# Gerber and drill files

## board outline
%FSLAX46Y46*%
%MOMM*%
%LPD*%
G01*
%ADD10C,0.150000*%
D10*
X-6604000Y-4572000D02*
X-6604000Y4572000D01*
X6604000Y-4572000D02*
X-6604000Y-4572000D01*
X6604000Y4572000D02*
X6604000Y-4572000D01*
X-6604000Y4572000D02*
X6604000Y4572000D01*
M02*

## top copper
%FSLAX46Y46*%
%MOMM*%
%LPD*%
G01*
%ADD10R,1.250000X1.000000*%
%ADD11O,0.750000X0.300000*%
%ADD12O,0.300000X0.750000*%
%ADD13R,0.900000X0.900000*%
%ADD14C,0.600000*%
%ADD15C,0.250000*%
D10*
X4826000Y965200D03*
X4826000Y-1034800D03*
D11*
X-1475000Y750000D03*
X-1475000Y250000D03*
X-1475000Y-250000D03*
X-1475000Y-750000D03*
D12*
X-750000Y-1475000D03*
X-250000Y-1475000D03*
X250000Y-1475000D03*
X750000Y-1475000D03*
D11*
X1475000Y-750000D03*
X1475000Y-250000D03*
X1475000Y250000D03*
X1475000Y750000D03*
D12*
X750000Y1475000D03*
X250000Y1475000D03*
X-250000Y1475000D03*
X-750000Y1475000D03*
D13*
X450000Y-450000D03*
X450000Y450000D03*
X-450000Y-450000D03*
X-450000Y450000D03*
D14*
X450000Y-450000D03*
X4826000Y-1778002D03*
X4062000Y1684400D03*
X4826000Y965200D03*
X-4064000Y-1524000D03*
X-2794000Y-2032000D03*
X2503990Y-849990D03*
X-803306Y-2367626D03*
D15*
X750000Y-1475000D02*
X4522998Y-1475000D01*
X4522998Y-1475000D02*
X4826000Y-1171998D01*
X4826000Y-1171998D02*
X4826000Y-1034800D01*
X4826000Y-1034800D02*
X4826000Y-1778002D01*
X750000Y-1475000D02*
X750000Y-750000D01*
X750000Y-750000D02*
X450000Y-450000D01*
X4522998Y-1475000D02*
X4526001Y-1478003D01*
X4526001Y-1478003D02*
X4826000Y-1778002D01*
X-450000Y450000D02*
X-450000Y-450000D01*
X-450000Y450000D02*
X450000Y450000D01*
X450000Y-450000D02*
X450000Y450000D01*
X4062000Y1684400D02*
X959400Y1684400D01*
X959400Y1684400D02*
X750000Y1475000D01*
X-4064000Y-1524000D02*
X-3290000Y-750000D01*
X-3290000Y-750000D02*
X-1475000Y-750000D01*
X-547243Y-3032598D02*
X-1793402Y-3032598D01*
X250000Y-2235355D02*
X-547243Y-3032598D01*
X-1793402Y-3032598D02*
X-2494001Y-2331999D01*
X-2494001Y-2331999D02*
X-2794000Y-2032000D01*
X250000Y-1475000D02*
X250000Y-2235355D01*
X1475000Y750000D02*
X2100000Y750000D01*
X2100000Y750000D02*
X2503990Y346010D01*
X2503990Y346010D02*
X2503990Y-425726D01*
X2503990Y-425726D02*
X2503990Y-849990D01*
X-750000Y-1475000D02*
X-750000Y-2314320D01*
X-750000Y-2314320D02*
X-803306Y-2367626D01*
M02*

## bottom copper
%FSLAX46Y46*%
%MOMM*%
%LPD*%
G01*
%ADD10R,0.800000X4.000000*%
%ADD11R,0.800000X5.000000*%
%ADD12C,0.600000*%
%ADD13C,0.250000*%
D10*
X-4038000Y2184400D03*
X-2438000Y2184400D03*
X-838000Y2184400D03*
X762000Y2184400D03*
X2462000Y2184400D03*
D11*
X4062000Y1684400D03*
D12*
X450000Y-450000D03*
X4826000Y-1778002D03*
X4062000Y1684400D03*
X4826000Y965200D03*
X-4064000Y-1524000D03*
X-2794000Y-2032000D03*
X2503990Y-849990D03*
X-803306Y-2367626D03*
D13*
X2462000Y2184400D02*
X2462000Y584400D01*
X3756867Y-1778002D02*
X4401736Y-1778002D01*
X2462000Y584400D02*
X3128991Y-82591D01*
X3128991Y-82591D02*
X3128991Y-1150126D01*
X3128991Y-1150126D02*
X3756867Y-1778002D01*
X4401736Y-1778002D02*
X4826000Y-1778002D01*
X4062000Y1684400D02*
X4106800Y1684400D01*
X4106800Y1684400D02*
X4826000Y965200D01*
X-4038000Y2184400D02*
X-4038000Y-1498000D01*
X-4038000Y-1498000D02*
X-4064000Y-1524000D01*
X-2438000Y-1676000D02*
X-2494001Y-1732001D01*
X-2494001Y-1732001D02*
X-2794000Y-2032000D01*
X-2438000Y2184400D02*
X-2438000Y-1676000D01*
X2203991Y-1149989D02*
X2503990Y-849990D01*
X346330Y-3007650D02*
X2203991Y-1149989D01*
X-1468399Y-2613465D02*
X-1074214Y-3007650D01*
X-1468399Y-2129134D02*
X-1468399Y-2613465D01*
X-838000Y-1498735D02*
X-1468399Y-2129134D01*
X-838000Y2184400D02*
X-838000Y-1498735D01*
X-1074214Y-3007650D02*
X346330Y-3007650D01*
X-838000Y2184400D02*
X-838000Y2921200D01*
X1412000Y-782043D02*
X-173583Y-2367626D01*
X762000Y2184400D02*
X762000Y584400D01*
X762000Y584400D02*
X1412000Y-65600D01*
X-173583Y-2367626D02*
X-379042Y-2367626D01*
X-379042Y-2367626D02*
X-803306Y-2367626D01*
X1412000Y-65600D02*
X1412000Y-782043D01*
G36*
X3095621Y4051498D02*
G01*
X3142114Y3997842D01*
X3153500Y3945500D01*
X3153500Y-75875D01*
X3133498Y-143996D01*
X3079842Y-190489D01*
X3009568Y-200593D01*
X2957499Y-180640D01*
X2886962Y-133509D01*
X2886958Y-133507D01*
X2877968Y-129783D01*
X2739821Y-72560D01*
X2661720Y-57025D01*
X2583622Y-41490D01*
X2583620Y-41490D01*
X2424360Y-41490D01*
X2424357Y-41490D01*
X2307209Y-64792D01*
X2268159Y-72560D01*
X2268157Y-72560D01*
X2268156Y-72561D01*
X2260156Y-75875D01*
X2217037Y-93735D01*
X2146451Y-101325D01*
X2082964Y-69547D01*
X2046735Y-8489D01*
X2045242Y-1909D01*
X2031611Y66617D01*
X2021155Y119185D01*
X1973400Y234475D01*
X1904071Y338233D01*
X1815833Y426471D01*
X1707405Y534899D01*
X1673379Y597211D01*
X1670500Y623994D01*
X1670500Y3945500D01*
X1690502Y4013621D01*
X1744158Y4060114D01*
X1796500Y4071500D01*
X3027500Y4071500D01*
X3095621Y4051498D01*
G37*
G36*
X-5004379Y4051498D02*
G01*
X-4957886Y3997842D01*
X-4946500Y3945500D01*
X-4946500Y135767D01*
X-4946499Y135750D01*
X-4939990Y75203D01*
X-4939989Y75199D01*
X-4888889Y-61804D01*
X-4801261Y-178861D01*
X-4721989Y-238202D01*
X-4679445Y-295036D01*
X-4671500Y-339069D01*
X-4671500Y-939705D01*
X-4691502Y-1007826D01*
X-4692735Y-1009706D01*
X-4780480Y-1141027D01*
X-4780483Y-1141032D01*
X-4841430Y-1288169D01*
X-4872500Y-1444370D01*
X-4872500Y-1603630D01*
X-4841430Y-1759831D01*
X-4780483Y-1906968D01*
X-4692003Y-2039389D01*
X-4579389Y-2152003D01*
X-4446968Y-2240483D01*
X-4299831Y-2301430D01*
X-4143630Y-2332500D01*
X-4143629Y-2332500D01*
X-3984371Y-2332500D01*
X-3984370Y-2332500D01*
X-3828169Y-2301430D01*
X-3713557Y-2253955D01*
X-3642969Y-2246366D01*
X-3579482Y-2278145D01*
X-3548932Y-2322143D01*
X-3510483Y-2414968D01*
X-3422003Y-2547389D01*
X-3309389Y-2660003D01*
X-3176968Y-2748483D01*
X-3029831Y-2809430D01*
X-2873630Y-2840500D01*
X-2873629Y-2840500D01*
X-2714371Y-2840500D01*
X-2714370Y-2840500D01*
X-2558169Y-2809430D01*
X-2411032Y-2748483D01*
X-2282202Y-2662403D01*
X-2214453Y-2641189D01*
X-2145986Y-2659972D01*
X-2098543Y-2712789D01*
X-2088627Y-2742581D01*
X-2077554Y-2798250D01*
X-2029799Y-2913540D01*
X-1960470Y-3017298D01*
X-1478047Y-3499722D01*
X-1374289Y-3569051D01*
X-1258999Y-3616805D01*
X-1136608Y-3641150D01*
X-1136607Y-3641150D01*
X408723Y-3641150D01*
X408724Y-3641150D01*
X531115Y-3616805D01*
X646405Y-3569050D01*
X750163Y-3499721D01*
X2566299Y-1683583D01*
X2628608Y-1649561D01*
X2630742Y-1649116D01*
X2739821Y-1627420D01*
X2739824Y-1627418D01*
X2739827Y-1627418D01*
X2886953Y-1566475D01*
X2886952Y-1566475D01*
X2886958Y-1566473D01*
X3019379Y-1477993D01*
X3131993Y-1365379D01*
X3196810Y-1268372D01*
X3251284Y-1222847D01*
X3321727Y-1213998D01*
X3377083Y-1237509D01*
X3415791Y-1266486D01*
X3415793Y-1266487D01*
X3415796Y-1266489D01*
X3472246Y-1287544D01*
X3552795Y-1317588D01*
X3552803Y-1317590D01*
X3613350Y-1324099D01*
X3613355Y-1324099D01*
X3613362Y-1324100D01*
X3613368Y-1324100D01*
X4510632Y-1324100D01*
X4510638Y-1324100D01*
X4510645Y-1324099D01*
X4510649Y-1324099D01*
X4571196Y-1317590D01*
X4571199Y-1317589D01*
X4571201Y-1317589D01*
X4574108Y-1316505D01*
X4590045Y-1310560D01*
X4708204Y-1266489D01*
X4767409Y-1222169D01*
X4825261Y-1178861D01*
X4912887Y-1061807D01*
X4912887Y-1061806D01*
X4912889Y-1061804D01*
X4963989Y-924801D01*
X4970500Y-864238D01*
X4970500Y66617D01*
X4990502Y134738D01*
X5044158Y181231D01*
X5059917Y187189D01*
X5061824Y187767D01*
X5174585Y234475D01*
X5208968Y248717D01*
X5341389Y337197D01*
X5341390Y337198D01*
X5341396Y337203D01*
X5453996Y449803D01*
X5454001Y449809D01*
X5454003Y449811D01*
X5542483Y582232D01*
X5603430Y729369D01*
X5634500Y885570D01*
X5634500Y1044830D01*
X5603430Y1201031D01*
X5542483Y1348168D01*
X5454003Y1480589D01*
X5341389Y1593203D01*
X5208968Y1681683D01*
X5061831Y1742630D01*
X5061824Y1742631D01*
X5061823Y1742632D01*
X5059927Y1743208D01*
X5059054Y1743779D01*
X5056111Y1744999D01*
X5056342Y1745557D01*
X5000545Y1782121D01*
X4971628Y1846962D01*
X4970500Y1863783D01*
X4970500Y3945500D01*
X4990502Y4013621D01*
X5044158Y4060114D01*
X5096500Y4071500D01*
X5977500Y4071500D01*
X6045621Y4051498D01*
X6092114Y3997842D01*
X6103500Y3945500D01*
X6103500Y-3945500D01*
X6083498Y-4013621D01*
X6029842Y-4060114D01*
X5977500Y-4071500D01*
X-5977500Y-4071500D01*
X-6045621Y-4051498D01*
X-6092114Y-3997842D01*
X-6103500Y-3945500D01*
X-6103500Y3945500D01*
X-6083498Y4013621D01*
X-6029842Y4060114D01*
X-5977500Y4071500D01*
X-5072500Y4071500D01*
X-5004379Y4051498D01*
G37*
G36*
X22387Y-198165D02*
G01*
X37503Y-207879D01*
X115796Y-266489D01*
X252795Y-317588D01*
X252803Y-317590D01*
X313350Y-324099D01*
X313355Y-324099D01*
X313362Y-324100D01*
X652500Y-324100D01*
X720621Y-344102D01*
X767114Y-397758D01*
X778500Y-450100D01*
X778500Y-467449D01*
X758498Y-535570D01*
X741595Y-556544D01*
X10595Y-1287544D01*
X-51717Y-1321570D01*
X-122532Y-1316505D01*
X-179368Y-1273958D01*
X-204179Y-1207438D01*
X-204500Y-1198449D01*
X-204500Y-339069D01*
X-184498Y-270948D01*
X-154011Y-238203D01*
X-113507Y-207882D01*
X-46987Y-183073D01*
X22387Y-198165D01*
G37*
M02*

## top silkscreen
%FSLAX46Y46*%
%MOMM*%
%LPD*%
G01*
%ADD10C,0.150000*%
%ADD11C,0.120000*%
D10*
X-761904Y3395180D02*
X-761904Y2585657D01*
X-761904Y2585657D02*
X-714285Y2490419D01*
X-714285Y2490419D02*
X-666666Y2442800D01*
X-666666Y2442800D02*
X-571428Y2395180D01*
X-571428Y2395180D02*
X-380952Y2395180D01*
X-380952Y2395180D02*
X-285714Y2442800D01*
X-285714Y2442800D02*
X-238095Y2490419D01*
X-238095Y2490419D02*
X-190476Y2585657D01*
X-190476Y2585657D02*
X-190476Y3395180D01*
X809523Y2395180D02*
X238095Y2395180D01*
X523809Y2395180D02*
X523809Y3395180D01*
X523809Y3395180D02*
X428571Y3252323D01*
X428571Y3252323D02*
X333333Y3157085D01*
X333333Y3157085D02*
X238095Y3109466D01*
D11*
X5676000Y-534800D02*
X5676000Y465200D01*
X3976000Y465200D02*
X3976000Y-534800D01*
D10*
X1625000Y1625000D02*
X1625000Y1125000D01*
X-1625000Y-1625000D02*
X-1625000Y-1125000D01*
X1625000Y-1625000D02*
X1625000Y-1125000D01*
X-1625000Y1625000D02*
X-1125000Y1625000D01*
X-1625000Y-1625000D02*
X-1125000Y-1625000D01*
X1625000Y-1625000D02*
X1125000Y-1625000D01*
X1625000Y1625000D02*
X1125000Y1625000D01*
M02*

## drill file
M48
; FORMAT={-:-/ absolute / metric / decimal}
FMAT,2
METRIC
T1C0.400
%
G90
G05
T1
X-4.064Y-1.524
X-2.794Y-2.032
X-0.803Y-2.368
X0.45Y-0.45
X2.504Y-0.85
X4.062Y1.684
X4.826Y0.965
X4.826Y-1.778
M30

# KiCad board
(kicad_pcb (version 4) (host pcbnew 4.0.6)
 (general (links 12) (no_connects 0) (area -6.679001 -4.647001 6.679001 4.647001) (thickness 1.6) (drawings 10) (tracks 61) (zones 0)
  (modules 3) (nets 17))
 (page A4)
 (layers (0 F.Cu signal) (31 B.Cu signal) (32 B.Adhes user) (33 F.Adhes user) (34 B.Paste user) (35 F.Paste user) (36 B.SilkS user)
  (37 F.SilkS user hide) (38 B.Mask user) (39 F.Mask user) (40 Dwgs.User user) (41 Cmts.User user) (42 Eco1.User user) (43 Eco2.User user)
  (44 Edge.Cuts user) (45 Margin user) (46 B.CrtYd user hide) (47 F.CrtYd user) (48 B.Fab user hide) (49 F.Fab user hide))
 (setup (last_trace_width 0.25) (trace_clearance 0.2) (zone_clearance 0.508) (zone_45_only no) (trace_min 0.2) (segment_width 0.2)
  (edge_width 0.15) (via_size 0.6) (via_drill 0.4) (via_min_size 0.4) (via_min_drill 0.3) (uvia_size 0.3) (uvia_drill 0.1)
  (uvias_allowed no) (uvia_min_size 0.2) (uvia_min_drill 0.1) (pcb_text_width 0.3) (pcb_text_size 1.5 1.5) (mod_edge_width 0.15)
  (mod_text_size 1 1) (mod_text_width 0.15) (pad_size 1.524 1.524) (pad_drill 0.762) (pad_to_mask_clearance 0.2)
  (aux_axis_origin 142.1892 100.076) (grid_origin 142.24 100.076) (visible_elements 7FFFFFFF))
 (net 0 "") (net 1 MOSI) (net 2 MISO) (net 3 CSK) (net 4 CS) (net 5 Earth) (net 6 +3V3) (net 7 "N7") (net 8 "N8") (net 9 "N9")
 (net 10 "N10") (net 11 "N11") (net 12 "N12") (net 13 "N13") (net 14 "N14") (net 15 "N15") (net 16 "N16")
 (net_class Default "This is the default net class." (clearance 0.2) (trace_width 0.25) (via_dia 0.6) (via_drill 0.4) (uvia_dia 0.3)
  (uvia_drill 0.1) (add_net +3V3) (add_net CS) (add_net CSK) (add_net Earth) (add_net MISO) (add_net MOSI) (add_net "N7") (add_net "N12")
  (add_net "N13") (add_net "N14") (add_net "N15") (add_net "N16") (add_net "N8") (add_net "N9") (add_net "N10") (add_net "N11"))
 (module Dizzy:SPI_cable (layer B.Cu) (at -4.438 -0.1844)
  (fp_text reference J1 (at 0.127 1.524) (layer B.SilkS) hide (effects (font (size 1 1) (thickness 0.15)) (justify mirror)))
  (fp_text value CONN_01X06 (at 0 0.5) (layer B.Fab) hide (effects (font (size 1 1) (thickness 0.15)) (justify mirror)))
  (pad 1 smd rect (at 0.4 -2) (size 0.8 4) (layers B.Cu B.Paste B.Mask) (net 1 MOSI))
  (pad 2 smd rect (at 2 -2) (size 0.8 4) (layers B.Cu B.Paste B.Mask) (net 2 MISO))
  (pad 3 smd rect (at 3.6 -2) (size 0.8 4) (layers B.Cu B.Paste B.Mask) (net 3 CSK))
  (pad 4 smd rect (at 5.2 -2) (size 0.8 4) (layers B.Cu B.Paste B.Mask) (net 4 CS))
  (pad 5 smd rect (at 6.9 -2) (size 0.8 4) (layers B.Cu B.Paste B.Mask) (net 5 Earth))
  (pad 6 smd rect (at 8.5 -1.5) (size 0.8 5) (layers B.Cu B.Paste B.Mask) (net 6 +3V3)))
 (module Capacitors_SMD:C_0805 (layer F.Cu) (at 4.826 0.0348 270)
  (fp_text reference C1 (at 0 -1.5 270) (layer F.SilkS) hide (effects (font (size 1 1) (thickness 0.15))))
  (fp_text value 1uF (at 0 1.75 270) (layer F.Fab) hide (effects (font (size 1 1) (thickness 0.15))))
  (fp_line (start 0.5 -0.85) (end -0.5 -0.85) (layer F.SilkS) (width 0.12))
  (fp_line (start -0.5 0.85) (end 0.5 0.85) (layer F.SilkS) (width 0.12))
  (pad 1 smd rect (at -1 0 270) (size 1 1.25) (layers F.Cu F.Paste F.Mask) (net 6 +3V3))
  (pad 2 smd rect (at 1 0 270) (size 1 1.25) (layers F.Cu F.Paste F.Mask) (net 5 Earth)))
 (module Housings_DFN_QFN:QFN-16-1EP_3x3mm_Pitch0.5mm (layer F.Cu) (at 0 0)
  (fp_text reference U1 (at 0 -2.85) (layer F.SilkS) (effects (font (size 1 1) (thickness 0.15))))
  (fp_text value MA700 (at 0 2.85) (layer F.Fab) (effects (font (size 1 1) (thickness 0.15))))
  (fp_line (start 1.625 -1.625) (end 1.625 -1.125) (layer F.SilkS) (width 0.15))
  (fp_line (start -1.625 1.625) (end -1.625 1.125) (layer F.SilkS) (width 0.15))
  (fp_line (start 1.625 1.625) (end 1.625 1.125) (layer F.SilkS) (width 0.15))
  (fp_line (start -1.625 -1.625) (end -1.125 -1.625) (layer F.SilkS) (width 0.15))
  (fp_line (start -1.625 1.625) (end -1.125 1.625) (layer F.SilkS) (width 0.15))
  (fp_line (start 1.625 1.625) (end 1.125 1.625) (layer F.SilkS) (width 0.15))
  (fp_line (start 1.625 -1.625) (end 1.125 -1.625) (layer F.SilkS) (width 0.15))
  (pad 1 smd oval (at -1.475 -0.75) (size 0.75 0.3) (layers F.Cu F.Paste F.Mask) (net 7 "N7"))
  (pad 2 smd oval (at -1.475 -0.25) (size 0.75 0.3) (layers F.Cu F.Paste F.Mask) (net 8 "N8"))
  (pad 3 smd oval (at -1.475 0.25) (size 0.75 0.3) (layers F.Cu F.Paste F.Mask) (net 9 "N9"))
  (pad 4 smd oval (at -1.475 0.75) (size 0.75 0.3) (layers F.Cu F.Paste F.Mask) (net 1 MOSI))
  (pad 5 smd oval (at -0.75 1.475 90) (size 0.75 0.3) (layers F.Cu F.Paste F.Mask) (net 4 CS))
  (pad 6 smd oval (at -0.25 1.475 90) (size 0.75 0.3) (layers F.Cu F.Paste F.Mask) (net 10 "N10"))
  (pad 7 smd oval (at 0.25 1.475 90) (size 0.75 0.3) (layers F.Cu F.Paste F.Mask) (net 2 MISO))
  (pad 8 smd oval (at 0.75 1.475 90) (size 0.75 0.3) (layers F.Cu F.Paste F.Mask) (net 5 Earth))
  (pad 9 smd oval (at 1.475 0.75) (size 0.75 0.3) (layers F.Cu F.Paste F.Mask) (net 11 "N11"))
  (pad 10 smd oval (at 1.475 0.25) (size 0.75 0.3) (layers F.Cu F.Paste F.Mask) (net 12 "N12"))
  (pad 11 smd oval (at 1.475 -0.25) (size 0.75 0.3) (layers F.Cu F.Paste F.Mask) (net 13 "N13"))
  (pad 12 smd oval (at 1.475 -0.75) (size 0.75 0.3) (layers F.Cu F.Paste F.Mask) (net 3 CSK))
  (pad 13 smd oval (at 0.75 -1.475 90) (size 0.75 0.3) (layers F.Cu F.Paste F.Mask) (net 6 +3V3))
  (pad 14 smd oval (at 0.25 -1.475 90) (size 0.75 0.3) (layers F.Cu F.Paste F.Mask) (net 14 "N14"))
  (pad 15 smd oval (at -0.25 -1.475 90) (size 0.75 0.3) (layers F.Cu F.Paste F.Mask) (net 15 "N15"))
  (pad 16 smd oval (at -0.75 -1.475 90) (size 0.75 0.3) (layers F.Cu F.Paste F.Mask) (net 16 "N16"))
  (pad 17 smd rect (at 0.45 0.45) (size 0.9 0.9) (layers F.Cu F.Paste F.Mask) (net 5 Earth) (solder_paste_margin_ratio -0.2))
  (pad 17 smd rect (at 0.45 -0.45) (size 0.9 0.9) (layers F.Cu F.Paste F.Mask) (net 5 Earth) (solder_paste_margin_ratio -0.2))
  (pad 17 smd rect (at -0.45 0.45) (size 0.9 0.9) (layers F.Cu F.Paste F.Mask) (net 5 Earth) (solder_paste_margin_ratio -0.2))
  (pad 17 smd rect (at -0.45 -0.45) (size 0.9 0.9) (layers F.Cu F.Paste F.Mask) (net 5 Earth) (solder_paste_margin_ratio -0.2)))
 (gr_line (start -6.604 4.572) (end -6.604 -4.572) (layer Edge.Cuts) (width 0.15))
 (gr_line (start 6.604 4.572) (end -6.604 4.572) (layer Edge.Cuts) (width 0.15))
 (gr_line (start 6.604 -4.572) (end 6.604 4.572) (layer Edge.Cuts) (width 0.15))
 (gr_line (start -6.604 -4.572) (end 6.604 -4.572) (layer Edge.Cuts) (width 0.15))
 (segment (start 0.75 1.475) (end 4.522998 1.475) (width 0.25) (layer F.Cu) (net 5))
 (segment (start 2.462 -2.1844) (end 2.462 -0.5844) (width 0.25) (layer B.Cu) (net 5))
 (segment (start 3.756867 1.778002) (end 4.401736 1.778002) (width 0.25) (layer B.Cu) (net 5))
 (segment (start 2.462 -0.5844) (end 3.128991 0.082591) (width 0.25) (layer B.Cu) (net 5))
 (segment (start 3.128991 0.082591) (end 3.128991 1.150126) (width 0.25) (layer B.Cu) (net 5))
 (segment (start 3.128991 1.150126) (end 3.756867 1.778002) (width 0.25) (layer B.Cu) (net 5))
 (segment (start 4.401736 1.778002) (end 4.826 1.778002) (width 0.25) (layer B.Cu) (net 5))
 (segment (start 4.522998 1.475) (end 4.826 1.171998) (width 0.25) (layer F.Cu) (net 5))
 (segment (start 4.826 1.171998) (end 4.826 1.0348) (width 0.25) (layer F.Cu) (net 5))
 (segment (start 4.826 1.0348) (end 4.826 1.778002) (width 0.25) (layer F.Cu) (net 5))
 (segment (start 0.75 1.475) (end 0.75 0.75) (width 0.25) (layer F.Cu) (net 5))
 (segment (start 0.75 0.75) (end 0.45 0.45) (width 0.25) (layer F.Cu) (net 5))
 (via (at 0.45 0.45) (size 0.6) (drill 0.4) (layers F.Cu B.Cu) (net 5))
 (segment (start 4.522998 1.475) (end 4.526001 1.478003) (width 0.25) (layer F.Cu) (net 5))
 (segment (start 4.526001 1.478003) (end 4.826 1.778002) (width 0.25) (layer F.Cu) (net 5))
 (via (at 4.826 1.778002) (size 0.6) (drill 0.4) (layers F.Cu B.Cu) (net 5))
 (segment (start -0.45 -0.45) (end -0.45 0.45) (width 0.25) (layer F.Cu) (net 5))
 (segment (start -0.45 -0.45) (end 0.45 -0.45) (width 0.25) (layer F.Cu) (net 5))
 (segment (start 0.45 0.45) (end 0.45 -0.45) (width 0.25) (layer F.Cu) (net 5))
 (segment (start 4.062 -1.6844) (end 0.9594 -1.6844) (width 0.25) (layer F.Cu) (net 6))
 (segment (start 0.9594 -1.6844) (end 0.75 -1.475) (width 0.25) (layer F.Cu) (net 6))
 (via (at 4.062 -1.6844) (size 0.6) (drill 0.4) (layers F.Cu B.Cu) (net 6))
 (segment (start 4.062 -1.6844) (end 4.1068 -1.6844) (width 0.25) (layer B.Cu) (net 6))
 (via (at 4.826 -0.9652) (size 0.6) (drill 0.4) (layers F.Cu B.Cu) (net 6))
 (segment (start 4.1068 -1.6844) (end 4.826 -0.9652) (width 0.25) (layer B.Cu) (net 6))
 (segment (start -4.064 1.524) (end -3.29 0.75) (width 0.25) (layer F.Cu) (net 1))
 (segment (start -3.29 0.75) (end -1.475 0.75) (width 0.25) (layer F.Cu) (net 1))
 (segment (start -4.038 -2.1844) (end -4.038 1.498) (width 0.25) (layer B.Cu) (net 1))
 (segment (start -4.038 1.498) (end -4.064 1.524) (width 0.25) (layer B.Cu) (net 1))
 (via (at -4.064 1.524) (size 0.6) (drill 0.4) (layers F.Cu B.Cu) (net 1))
 (segment (start -0.547243 3.032598) (end -1.793402 3.032598) (width 0.25) (layer F.Cu) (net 2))
 (segment (start 0.25 2.235355) (end -0.547243 3.032598) (width 0.25) (layer F.Cu) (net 2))
 (segment (start -1.793402 3.032598) (end -2.494001 2.331999) (width 0.25) (layer F.Cu) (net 2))
 (segment (start -2.494001 2.331999) (end -2.794 2.032) (width 0.25) (layer F.Cu) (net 2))
 (segment (start 0.25 1.475) (end 0.25 2.235355) (width 0.25) (layer F.Cu) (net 2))
 (segment (start -2.438 1.676) (end -2.494001 1.732001) (width 0.25) (layer B.Cu) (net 2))
 (segment (start -2.494001 1.732001) (end -2.794 2.032) (width 0.25) (layer B.Cu) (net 2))
 (segment (start -2.438 -2.1844) (end -2.438 1.676) (width 0.25) (layer B.Cu) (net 2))
 (via (at -2.794 2.032) (size 0.6) (drill 0.4) (layers F.Cu B.Cu) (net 2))
 (segment (start 1.475 -0.75) (end 2.1 -0.75) (width 0.25) (layer F.Cu) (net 3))
 (segment (start 2.203991 1.149989) (end 2.50399 0.84999) (width 0.25) (layer B.Cu) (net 3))
 (segment (start 0.34633 3.00765) (end 2.203991 1.149989) (width 0.25) (layer B.Cu) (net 3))
 (segment (start 2.1 -0.75) (end 2.50399 -0.34601) (width 0.25) (layer F.Cu) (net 3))
 (segment (start 2.50399 -0.34601) (end 2.50399 0.425726) (width 0.25) (layer F.Cu) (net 3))
 (segment (start -1.468399 2.613465) (end -1.074214 3.00765) (width 0.25) (layer B.Cu) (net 3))
 (segment (start -1.468399 2.129134) (end -1.468399 2.613465) (width 0.25) (layer B.Cu) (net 3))
 (segment (start -0.838 1.498735) (end -1.468399 2.129134) (width 0.25) (layer B.Cu) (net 3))
 (segment (start -0.838 -2.1844) (end -0.838 1.498735) (width 0.25) (layer B.Cu) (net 3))
 (segment (start -1.074214 3.00765) (end 0.34633 3.00765) (width 0.25) (layer B.Cu) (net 3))
 (segment (start 2.50399 0.425726) (end 2.50399 0.84999) (width 0.25) (layer F.Cu) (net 3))
 (via (at 2.50399 0.84999) (size 0.6) (drill 0.4) (layers F.Cu B.Cu) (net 3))
 (segment (start -0.838 -2.1844) (end -0.838 -2.9212) (width 0.25) (layer B.Cu) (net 3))
 (segment (start -0.75 1.475) (end -0.75 2.31432) (width 0.25) (layer F.Cu) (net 4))
 (segment (start -0.75 2.31432) (end -0.803306 2.367626) (width 0.25) (layer F.Cu) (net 4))
 (segment (start 1.412 0.782043) (end -0.173583 2.367626) (width 0.25) (layer B.Cu) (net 4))
 (via (at -0.803306 2.367626) (size 0.6) (drill 0.4) (layers F.Cu B.Cu) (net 4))
 (segment (start 0.762 -2.1844) (end 0.762 -0.5844) (width 0.25) (layer B.Cu) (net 4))
 (segment (start 0.762 -0.5844) (end 1.412 0.0656) (width 0.25) (layer B.Cu) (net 4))
 (segment (start -0.173583 2.367626) (end -0.379042 2.367626) (width 0.25) (layer B.Cu) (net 4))
 (segment (start -0.379042 2.367626) (end -0.803306 2.367626) (width 0.25) (layer B.Cu) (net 4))
 (segment (start 1.412 0.0656) (end 1.412 0.782043) (width 0.25) (layer B.Cu) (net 4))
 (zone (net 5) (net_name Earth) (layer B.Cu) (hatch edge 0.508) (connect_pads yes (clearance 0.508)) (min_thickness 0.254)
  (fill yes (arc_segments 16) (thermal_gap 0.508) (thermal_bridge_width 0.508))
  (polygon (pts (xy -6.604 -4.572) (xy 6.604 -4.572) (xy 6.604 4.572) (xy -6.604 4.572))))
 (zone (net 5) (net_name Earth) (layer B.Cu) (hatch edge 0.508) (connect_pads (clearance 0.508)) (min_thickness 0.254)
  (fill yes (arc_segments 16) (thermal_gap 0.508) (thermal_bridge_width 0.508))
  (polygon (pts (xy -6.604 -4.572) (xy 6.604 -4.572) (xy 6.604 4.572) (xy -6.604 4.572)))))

